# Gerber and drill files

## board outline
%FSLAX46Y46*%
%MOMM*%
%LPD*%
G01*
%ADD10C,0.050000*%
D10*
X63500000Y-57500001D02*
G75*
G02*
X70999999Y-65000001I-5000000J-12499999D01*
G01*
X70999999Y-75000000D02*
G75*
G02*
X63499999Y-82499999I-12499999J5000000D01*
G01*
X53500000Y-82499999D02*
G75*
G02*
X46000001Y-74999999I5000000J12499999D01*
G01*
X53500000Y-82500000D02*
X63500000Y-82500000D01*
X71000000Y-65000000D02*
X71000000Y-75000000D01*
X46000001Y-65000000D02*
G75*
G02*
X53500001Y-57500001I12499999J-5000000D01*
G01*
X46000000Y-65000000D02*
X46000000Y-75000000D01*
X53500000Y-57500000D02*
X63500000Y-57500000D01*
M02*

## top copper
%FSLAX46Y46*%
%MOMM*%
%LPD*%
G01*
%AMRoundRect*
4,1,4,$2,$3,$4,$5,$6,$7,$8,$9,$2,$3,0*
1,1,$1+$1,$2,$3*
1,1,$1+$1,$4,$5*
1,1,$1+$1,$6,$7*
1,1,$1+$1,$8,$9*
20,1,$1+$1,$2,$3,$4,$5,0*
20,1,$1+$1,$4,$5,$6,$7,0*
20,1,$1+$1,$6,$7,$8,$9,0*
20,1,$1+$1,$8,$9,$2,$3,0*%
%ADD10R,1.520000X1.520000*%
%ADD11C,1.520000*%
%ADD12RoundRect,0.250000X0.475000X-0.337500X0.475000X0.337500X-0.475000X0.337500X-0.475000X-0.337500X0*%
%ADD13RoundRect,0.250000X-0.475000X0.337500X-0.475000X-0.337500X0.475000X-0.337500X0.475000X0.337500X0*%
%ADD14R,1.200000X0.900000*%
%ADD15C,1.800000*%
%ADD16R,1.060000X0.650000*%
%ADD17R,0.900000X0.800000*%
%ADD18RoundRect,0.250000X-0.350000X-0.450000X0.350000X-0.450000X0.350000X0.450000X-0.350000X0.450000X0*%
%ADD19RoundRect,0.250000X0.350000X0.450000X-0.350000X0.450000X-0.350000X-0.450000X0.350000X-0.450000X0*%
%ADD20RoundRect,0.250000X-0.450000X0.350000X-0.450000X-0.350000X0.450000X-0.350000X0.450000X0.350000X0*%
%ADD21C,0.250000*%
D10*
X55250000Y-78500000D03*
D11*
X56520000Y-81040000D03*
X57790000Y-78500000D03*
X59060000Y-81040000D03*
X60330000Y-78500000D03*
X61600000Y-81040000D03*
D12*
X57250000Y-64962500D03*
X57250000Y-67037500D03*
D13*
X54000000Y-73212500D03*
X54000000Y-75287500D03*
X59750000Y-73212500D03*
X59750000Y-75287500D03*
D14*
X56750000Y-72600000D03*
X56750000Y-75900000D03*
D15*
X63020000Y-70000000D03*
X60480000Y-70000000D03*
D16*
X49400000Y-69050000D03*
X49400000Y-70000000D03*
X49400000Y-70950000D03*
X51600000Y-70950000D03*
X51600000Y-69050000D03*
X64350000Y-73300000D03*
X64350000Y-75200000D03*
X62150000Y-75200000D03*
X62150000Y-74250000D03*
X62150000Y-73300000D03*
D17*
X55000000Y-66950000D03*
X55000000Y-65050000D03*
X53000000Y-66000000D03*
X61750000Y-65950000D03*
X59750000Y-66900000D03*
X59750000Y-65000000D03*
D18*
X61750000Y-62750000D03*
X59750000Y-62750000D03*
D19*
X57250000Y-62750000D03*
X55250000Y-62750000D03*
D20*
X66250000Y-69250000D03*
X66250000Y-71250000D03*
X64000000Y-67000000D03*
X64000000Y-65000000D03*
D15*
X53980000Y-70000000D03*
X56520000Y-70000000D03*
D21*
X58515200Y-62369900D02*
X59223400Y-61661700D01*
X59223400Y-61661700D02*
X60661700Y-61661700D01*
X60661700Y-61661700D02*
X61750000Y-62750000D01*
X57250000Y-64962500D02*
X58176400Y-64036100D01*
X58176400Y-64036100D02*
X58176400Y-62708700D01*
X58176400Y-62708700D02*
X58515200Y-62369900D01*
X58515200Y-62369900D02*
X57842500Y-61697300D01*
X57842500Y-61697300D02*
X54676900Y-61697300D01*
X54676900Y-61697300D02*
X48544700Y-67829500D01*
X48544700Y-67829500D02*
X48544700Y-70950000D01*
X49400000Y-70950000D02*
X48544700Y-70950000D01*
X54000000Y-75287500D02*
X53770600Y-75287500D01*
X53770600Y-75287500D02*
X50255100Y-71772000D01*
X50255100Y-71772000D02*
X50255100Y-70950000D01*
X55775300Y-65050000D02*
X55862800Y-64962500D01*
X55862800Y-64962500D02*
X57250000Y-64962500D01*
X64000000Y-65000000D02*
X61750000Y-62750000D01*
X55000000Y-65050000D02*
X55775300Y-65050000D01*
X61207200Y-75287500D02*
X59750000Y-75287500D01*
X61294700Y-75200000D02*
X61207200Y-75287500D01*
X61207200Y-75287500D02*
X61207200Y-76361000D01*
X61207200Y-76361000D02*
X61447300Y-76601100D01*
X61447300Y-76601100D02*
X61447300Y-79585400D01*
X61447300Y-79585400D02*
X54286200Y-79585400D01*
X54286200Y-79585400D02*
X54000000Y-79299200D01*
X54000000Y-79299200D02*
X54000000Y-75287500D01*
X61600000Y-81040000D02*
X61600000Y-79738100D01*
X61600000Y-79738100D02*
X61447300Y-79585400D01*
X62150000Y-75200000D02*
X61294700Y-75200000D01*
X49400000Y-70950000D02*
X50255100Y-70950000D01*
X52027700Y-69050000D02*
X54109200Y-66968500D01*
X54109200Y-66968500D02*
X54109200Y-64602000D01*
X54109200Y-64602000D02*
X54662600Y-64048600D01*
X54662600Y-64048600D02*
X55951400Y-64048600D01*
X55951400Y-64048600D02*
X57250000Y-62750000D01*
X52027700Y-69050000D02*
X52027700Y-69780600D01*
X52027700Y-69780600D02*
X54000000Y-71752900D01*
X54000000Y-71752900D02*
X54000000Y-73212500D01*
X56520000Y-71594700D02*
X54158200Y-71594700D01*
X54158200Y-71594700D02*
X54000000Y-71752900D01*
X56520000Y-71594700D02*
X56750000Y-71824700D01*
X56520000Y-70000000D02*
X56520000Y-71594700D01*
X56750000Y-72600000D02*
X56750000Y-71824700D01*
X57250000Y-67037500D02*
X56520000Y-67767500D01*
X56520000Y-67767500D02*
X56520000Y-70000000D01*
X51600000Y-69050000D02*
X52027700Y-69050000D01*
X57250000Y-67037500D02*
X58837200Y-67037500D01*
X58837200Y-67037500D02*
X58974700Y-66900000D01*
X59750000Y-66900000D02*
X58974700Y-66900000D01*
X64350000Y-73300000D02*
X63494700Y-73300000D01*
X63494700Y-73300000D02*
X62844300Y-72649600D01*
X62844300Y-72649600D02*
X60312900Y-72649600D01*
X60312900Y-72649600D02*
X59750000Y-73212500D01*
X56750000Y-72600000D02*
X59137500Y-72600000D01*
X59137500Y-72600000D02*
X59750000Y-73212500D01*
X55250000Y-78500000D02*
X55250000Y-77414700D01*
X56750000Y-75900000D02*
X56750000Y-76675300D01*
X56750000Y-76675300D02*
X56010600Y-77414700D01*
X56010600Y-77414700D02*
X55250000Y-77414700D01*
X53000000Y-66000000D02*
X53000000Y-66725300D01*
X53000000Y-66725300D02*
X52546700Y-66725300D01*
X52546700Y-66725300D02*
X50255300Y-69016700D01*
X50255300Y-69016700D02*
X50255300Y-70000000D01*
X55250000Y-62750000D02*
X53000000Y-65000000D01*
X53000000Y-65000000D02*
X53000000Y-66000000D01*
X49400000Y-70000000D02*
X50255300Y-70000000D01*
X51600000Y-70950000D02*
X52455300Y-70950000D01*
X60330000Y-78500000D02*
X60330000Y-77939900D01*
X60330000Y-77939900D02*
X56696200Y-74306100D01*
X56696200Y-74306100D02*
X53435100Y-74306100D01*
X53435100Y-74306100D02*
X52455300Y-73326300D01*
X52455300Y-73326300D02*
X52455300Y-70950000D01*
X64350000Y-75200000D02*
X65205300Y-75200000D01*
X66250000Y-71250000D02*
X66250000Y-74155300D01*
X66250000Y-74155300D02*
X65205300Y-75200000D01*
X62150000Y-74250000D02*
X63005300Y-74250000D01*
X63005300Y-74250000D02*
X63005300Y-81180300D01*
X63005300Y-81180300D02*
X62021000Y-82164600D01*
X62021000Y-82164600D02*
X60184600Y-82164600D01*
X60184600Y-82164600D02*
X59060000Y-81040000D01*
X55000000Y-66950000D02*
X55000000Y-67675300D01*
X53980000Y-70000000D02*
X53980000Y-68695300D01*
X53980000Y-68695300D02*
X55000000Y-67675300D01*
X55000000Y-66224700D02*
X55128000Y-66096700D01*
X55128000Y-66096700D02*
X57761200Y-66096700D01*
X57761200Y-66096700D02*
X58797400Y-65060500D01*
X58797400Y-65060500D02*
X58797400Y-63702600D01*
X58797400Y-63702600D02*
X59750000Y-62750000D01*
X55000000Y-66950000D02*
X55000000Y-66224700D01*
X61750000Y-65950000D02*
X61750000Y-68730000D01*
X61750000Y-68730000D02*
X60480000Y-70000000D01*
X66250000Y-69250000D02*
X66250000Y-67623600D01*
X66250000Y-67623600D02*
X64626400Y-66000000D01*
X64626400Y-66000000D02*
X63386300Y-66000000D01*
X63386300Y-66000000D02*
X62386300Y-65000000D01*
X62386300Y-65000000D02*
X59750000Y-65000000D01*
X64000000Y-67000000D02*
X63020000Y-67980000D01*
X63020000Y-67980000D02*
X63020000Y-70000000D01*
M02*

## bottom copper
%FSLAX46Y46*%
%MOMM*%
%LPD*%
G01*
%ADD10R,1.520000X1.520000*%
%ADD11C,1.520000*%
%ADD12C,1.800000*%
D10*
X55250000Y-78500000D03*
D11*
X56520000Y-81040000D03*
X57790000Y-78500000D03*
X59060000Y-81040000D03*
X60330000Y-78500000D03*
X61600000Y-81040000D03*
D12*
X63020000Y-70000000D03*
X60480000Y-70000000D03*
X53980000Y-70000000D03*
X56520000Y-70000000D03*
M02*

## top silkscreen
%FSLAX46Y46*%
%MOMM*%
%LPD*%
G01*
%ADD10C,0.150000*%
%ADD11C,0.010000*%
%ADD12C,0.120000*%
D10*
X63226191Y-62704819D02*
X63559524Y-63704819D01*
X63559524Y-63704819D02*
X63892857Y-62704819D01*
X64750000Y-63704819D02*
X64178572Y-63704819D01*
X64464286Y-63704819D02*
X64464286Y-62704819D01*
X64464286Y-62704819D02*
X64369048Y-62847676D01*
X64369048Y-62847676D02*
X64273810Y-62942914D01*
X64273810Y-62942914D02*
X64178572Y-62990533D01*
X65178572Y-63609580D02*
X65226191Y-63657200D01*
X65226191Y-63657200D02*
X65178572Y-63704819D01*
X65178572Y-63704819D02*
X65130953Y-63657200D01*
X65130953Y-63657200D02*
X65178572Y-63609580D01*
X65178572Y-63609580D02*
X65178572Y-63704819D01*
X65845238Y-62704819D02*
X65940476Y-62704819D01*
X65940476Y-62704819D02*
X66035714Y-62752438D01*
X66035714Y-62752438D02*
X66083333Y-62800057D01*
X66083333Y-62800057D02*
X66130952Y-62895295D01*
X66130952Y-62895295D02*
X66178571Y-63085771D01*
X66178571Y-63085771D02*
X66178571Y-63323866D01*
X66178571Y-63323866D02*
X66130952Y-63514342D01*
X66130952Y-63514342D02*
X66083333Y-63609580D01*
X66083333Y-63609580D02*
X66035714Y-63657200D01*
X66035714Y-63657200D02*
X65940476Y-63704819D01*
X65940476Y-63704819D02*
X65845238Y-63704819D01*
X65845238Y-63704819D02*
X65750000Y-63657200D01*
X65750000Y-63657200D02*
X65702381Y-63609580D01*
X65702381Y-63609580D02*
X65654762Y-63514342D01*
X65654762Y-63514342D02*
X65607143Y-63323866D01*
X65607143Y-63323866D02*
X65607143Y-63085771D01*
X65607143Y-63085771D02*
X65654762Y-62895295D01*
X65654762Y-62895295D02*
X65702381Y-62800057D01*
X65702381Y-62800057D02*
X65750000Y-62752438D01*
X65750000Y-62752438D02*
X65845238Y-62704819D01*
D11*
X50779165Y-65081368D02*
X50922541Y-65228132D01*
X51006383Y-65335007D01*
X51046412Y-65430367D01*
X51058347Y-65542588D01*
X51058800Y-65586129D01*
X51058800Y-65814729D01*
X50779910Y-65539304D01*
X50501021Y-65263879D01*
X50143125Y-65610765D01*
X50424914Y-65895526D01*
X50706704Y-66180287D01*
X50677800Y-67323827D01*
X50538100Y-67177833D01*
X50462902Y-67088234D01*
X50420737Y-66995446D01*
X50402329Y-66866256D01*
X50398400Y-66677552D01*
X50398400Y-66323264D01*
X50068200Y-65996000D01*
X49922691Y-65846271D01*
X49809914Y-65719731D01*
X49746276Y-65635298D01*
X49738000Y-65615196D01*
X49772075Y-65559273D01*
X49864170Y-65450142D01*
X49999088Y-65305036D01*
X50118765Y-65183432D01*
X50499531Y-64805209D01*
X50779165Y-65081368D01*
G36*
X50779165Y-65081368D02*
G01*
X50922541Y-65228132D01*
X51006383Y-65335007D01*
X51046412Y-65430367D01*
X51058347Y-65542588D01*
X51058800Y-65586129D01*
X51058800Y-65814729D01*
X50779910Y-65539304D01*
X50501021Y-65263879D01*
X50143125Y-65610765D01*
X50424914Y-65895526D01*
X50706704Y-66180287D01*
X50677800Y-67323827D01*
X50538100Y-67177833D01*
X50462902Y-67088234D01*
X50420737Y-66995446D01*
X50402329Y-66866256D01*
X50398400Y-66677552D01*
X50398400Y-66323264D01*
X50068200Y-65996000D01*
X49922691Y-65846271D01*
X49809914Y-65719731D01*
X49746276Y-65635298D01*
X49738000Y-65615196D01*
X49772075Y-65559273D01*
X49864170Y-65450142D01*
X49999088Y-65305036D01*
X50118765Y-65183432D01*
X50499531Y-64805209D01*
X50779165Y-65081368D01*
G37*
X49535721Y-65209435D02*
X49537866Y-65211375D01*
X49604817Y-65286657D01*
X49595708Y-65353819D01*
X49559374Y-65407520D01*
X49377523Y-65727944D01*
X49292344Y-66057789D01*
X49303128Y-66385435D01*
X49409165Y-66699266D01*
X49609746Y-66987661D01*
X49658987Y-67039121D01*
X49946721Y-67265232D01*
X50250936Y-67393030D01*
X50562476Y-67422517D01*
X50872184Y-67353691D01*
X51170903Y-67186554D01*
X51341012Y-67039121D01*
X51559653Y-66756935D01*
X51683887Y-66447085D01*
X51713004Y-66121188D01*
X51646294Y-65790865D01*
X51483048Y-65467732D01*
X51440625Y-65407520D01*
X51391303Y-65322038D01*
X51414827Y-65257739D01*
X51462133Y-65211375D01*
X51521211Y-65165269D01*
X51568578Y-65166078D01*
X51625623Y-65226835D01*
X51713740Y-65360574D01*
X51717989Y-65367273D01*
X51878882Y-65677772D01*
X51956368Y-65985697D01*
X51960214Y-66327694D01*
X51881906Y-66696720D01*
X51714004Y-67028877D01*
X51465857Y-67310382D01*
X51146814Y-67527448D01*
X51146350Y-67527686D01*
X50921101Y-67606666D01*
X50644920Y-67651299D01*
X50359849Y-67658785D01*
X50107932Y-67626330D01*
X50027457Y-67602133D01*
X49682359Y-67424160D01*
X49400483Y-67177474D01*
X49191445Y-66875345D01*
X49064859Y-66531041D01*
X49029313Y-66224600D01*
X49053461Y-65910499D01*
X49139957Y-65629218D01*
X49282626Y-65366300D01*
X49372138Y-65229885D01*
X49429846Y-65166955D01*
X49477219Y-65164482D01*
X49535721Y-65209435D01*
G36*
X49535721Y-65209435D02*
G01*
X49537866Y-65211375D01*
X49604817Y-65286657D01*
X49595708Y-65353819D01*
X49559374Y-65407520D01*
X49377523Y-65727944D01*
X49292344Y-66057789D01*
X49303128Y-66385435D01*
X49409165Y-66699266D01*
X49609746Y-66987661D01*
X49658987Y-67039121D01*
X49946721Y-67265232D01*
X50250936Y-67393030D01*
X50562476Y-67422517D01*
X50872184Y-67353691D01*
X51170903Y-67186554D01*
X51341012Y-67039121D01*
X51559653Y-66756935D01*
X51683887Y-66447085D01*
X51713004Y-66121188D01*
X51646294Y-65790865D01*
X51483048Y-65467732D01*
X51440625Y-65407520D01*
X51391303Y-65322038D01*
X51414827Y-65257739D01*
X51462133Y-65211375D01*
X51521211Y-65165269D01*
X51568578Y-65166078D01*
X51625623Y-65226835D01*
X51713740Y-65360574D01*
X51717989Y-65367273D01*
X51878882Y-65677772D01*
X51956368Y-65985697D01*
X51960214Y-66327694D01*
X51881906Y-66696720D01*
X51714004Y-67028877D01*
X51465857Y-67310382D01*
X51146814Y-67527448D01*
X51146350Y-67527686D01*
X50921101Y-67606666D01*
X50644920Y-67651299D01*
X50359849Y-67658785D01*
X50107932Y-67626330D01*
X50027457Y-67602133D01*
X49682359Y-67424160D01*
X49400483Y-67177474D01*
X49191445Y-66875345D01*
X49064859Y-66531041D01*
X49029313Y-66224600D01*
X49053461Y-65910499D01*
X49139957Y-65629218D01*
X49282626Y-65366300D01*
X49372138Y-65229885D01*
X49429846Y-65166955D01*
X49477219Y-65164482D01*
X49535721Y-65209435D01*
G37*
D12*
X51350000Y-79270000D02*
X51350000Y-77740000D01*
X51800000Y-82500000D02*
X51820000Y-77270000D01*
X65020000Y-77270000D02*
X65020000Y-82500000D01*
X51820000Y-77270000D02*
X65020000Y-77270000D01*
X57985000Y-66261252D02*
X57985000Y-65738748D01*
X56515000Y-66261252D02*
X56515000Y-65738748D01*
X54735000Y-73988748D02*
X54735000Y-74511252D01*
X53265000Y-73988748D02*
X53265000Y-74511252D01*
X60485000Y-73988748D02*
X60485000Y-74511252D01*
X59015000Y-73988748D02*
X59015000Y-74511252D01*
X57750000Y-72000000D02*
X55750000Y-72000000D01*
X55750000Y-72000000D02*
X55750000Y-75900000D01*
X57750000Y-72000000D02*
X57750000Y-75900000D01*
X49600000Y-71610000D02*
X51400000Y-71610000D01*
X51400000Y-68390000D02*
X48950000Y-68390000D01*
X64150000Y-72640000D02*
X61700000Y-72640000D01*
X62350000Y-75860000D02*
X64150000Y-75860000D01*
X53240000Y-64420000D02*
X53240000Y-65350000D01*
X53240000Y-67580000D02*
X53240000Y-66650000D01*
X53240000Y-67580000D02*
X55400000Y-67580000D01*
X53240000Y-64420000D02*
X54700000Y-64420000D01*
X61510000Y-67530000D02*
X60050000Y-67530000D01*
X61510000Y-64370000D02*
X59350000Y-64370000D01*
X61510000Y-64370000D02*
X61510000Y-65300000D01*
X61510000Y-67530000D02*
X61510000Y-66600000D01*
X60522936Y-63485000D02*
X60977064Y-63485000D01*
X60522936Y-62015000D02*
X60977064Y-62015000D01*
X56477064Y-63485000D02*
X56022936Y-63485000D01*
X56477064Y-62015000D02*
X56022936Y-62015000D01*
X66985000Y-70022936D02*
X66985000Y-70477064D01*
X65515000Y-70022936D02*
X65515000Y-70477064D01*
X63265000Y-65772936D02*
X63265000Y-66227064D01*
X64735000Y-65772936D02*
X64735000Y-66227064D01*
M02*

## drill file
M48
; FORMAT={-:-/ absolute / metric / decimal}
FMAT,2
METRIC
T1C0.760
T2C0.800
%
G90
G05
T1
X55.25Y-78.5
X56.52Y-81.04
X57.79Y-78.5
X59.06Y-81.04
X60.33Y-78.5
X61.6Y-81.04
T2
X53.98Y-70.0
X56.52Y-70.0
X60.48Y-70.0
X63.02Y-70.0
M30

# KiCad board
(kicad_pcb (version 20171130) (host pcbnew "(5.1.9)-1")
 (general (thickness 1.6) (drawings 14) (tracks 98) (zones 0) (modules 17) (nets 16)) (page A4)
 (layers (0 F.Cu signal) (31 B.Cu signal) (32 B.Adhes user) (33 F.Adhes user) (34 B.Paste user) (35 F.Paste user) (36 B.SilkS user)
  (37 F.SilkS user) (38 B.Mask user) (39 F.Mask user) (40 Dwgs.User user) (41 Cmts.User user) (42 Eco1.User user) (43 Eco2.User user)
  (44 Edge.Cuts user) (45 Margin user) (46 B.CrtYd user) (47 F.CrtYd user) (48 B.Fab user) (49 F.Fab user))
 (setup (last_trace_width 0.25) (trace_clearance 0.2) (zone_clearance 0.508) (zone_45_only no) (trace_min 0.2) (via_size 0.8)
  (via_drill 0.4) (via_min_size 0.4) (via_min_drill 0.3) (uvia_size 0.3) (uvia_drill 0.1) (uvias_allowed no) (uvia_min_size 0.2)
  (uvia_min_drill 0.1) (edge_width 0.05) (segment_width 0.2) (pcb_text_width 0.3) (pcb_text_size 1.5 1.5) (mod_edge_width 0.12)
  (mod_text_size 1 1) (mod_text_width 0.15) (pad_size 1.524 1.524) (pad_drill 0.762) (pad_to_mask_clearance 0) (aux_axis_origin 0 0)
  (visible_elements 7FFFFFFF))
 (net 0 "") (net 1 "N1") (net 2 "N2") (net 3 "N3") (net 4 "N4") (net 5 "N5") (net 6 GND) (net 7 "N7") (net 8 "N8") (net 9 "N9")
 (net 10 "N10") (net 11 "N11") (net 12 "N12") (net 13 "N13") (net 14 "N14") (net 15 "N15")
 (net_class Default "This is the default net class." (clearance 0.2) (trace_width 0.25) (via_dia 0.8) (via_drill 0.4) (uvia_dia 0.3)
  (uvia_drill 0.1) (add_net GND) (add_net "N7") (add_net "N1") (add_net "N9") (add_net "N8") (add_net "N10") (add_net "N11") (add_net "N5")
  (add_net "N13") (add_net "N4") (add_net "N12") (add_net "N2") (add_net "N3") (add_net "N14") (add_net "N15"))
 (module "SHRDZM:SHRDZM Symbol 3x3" (layer F.Cu) (at 50.5 66.25)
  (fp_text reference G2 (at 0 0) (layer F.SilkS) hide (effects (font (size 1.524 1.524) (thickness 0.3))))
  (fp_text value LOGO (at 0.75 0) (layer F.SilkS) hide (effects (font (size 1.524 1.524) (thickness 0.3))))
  (fp_poly
   (pts (xy 0.279165 -1.168632) (xy 0.422541 -1.021868) (xy 0.506383 -0.914993) (xy 0.546412 -0.819633) (xy 0.558347 -0.707412)
    (xy 0.5588 -0.663871) (xy 0.5588 -0.435271) (xy 0.27991 -0.710696) (xy 0.001021 -0.986121) (xy -0.356875 -0.639235)
    (xy -0.075086 -0.354474) (xy 0.206704 -0.069713) (xy 0.1778 1.073827) (xy 0.0381 0.927833) (xy -0.037098 0.838234)
    (xy -0.079263 0.745446) (xy -0.097671 0.616256) (xy -0.1016 0.427552) (xy -0.1016 0.073264) (xy -0.4318 -0.254) (xy -0.577309 -0.403729)
    (xy -0.690086 -0.530269) (xy -0.753724 -0.614702) (xy -0.762 -0.634804) (xy -0.727925 -0.690727) (xy -0.63583 -0.799858)
    (xy -0.500912 -0.944964) (xy -0.381235 -1.066568) (xy -0.000469 -1.444791) (xy 0.279165 -1.168632))
   (layer F.SilkS) (width 0.01))
  (fp_poly
   (pts (xy -0.964279 -1.040565) (xy -0.962134 -1.038625) (xy -0.895183 -0.963343) (xy -0.904292 -0.896181) (xy -0.940626 -0.84248)
    (xy -1.122477 -0.522056) (xy -1.207656 -0.192211) (xy -1.196872 0.135435) (xy -1.090835 0.449266) (xy -0.890254 0.737661)
    (xy -0.841013 0.789121) (xy -0.553279 1.015232) (xy -0.249064 1.14303) (xy 0.062476 1.172517) (xy 0.372184 1.103691)
    (xy 0.670903 0.936554) (xy 0.841012 0.789121) (xy 1.059653 0.506935) (xy 1.183887 0.197085) (xy 1.213004 -0.128812)
    (xy 1.146294 -0.459135) (xy 0.983048 -0.782268) (xy 0.940625 -0.84248) (xy 0.891303 -0.927962) (xy 0.914827 -0.992261)
    (xy 0.962133 -1.038625) (xy 1.021211 -1.084731) (xy 1.068578 -1.083922) (xy 1.125623 -1.023165) (xy 1.21374 -0.889426)
    (xy 1.217989 -0.882727) (xy 1.378882 -0.572228) (xy 1.456368 -0.264303) (xy 1.460214 0.077694) (xy 1.381906 0.44672)
    (xy 1.214004 0.778877) (xy 0.965857 1.060382) (xy 0.646814 1.277448) (xy 0.64635 1.277686) (xy 0.421101 1.356666) (xy 0.14492 1.401299)
    (xy -0.140151 1.408785) (xy -0.392068 1.37633) (xy -0.472543 1.352133) (xy -0.817641 1.17416) (xy -1.099517 0.927474)
    (xy -1.308555 0.625345) (xy -1.435141 0.281041) (xy -1.470687 -0.0254) (xy -1.446539 -0.339501) (xy -1.360043 -0.620782)
    (xy -1.217374 -0.8837) (xy -1.127862 -1.020115) (xy -1.070154 -1.083045) (xy -1.022781 -1.085518) (xy -0.964279 -1.040565))
   (layer F.SilkS) (width 0.01)))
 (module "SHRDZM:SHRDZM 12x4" (layer B.Cu) (at 58.75 63.25 180)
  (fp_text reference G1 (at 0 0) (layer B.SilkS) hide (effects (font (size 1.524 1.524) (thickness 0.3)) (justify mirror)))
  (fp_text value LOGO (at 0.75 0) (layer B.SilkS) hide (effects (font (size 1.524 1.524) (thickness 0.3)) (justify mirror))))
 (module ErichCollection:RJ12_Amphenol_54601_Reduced (layer F.Cu) (at 55.25 78.5)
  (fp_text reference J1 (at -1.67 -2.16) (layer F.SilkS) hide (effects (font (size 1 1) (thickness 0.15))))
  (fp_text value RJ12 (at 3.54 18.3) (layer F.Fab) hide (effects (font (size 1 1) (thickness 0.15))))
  (fp_line (start -3.9 0.77) (end -3.9 -0.76) (layer F.SilkS) (width 0.12))
  (fp_line (start -3.45 4) (end -3.43 -1.23) (layer F.SilkS) (width 0.12))
  (fp_line (start 9.77 -1.23) (end 9.77 4) (layer F.SilkS) (width 0.12))
  (fp_line (start -3.43 -1.23) (end 9.77 -1.23) (layer F.SilkS) (width 0.12))
  (pad 1 thru_hole rect (at 0 0) (size 1.52 1.52) (drill 0.76) (layers *.Cu *.Mask) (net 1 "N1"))
  (pad 2 thru_hole circle (at 1.27 2.54) (size 1.52 1.52) (drill 0.76) (layers *.Cu *.Mask) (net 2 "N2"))
  (pad 3 thru_hole circle (at 2.54 0) (size 1.52 1.52) (drill 0.76) (layers *.Cu *.Mask) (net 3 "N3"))
  (pad 4 thru_hole circle (at 3.81 2.54) (size 1.52 1.52) (drill 0.76) (layers *.Cu *.Mask) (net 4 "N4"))
  (pad 5 thru_hole circle (at 5.08 0) (size 1.52 1.52) (drill 0.76) (layers *.Cu *.Mask) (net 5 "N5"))
  (pad 6 thru_hole circle (at 6.35 2.54) (size 1.52 1.52) (drill 0.76) (layers *.Cu *.Mask) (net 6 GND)))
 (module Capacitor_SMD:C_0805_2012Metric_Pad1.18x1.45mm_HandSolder (layer F.Cu) (at 57.25 66 90)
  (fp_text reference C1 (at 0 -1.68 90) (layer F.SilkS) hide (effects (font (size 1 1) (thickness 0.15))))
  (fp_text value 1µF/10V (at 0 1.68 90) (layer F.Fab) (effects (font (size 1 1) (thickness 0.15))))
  (fp_line (start -0.261252 0.735) (end 0.261252 0.735) (layer F.SilkS) (width 0.12))
  (fp_line (start -0.261252 -0.735) (end 0.261252 -0.735) (layer F.SilkS) (width 0.12))
  (pad 2 smd roundrect (at 1.0375 0 90) (size 1.175 1.45) (layers F.Cu F.Paste F.Mask) (roundrect_rratio 0.212766) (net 6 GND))
  (pad 1 smd roundrect (at -1.0375 0 90) (size 1.175 1.45) (layers F.Cu F.Paste F.Mask) (roundrect_rratio 0.212766) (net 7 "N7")))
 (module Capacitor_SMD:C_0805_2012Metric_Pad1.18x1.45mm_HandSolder (layer F.Cu) (at 54 74.25 270)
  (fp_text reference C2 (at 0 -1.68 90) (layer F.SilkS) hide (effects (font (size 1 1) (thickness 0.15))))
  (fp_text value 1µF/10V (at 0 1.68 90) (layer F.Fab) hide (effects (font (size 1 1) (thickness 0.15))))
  (fp_line (start -0.261252 -0.735) (end 0.261252 -0.735) (layer F.SilkS) (width 0.12))
  (fp_line (start -0.261252 0.735) (end 0.261252 0.735) (layer F.SilkS) (width 0.12))
  (pad 1 smd roundrect (at -1.0375 0 270) (size 1.175 1.45) (layers F.Cu F.Paste F.Mask) (roundrect_rratio 0.212766) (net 7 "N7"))
  (pad 2 smd roundrect (at 1.0375 0 270) (size 1.175 1.45) (layers F.Cu F.Paste F.Mask) (roundrect_rratio 0.212766) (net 6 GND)))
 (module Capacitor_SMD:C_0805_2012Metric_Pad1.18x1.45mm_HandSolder (layer F.Cu) (at 59.75 74.25 270)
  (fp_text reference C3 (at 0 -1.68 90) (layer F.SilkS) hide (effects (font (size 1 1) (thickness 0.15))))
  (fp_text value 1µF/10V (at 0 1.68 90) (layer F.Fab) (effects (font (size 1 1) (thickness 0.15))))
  (fp_line (start -0.261252 -0.735) (end 0.261252 -0.735) (layer F.SilkS) (width 0.12))
  (fp_line (start -0.261252 0.735) (end 0.261252 0.735) (layer F.SilkS) (width 0.12))
  (pad 1 smd roundrect (at -1.0375 0 270) (size 1.175 1.45) (layers F.Cu F.Paste F.Mask) (roundrect_rratio 0.212766) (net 7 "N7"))
  (pad 2 smd roundrect (at 1.0375 0 270) (size 1.175 1.45) (layers F.Cu F.Paste F.Mask) (roundrect_rratio 0.212766) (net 6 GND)))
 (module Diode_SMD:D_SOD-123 (layer F.Cu) (at 56.75 74.25 270)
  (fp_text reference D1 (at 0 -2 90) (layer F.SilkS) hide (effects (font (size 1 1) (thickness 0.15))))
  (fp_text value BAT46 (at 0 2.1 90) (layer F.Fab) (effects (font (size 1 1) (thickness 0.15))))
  (fp_line (start -2.25 -1) (end -2.25 1) (layer F.SilkS) (width 0.12))
  (fp_line (start -2.25 1) (end 1.65 1) (layer F.SilkS) (width 0.12))
  (fp_line (start -2.25 -1) (end 1.65 -1) (layer F.SilkS) (width 0.12))
  (pad 1 smd rect (at -1.65 0 270) (size 0.9 1.2) (layers F.Cu F.Paste F.Mask) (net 7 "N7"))
  (pad 2 smd rect (at 1.65 0 270) (size 0.9 1.2) (layers F.Cu F.Paste F.Mask) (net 1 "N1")))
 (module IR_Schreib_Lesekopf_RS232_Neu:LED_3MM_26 (layer F.Cu) (at 61.75 70 180)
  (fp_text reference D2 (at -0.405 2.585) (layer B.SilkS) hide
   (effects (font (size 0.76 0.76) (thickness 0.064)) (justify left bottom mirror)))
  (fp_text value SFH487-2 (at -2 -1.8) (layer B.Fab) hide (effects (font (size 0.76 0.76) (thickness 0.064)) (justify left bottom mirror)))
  (pad 2 thru_hole circle (at -1.27 0 180) (size 1.8 1.8) (drill 0.8) (layers *.Cu *.Mask) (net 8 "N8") (solder_mask_margin 0.1016))
  (pad 1 thru_hole circle (at 1.27 0 180) (size 1.8 1.8) (drill 0.8) (layers *.Cu *.Mask) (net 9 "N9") (solder_mask_margin 0.1016)))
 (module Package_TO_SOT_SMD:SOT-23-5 (layer F.Cu) (at 50.5 70)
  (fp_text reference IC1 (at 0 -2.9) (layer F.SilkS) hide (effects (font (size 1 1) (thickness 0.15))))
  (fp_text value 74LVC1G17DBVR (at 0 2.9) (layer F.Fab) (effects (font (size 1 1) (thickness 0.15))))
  (fp_line (start -0.9 1.61) (end 0.9 1.61) (layer F.SilkS) (width 0.12))
  (fp_line (start 0.9 -1.61) (end -1.55 -1.61) (layer F.SilkS) (width 0.12))
  (pad 1 smd rect (at -1.1 -0.95) (size 1.06 0.65) (layers F.Cu F.Paste F.Mask) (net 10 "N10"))
  (pad 2 smd rect (at -1.1 0) (size 1.06 0.65) (layers F.Cu F.Paste F.Mask) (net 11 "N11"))
  (pad 3 smd rect (at -1.1 0.95) (size 1.06 0.65) (layers F.Cu F.Paste F.Mask) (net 6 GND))
  (pad 4 smd rect (at 1.1 0.95) (size 1.06 0.65) (layers F.Cu F.Paste F.Mask) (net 5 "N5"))
  (pad 5 smd rect (at 1.1 -0.95) (size 1.06 0.65) (layers F.Cu F.Paste F.Mask) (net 7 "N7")))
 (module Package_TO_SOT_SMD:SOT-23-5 (layer F.Cu) (at 63.25 74.25)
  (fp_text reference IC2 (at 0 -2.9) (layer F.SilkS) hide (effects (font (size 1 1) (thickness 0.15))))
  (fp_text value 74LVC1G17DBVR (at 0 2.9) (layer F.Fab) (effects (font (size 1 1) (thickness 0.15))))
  (fp_line (start 0.9 -1.61) (end -1.55 -1.61) (layer F.SilkS) (width 0.12))
  (fp_line (start -0.9 1.61) (end 0.9 1.61) (layer F.SilkS) (width 0.12))
  (pad 5 smd rect (at 1.1 -0.95) (size 1.06 0.65) (layers F.Cu F.Paste F.Mask) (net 7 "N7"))
  (pad 4 smd rect (at 1.1 0.95) (size 1.06 0.65) (layers F.Cu F.Paste F.Mask) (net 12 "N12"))
  (pad 3 smd rect (at -1.1 0.95) (size 1.06 0.65) (layers F.Cu F.Paste F.Mask) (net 6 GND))
  (pad 2 smd rect (at -1.1 0) (size 1.06 0.65) (layers F.Cu F.Paste F.Mask) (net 4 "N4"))
  (pad 1 smd rect (at -1.1 -0.95) (size 1.06 0.65) (layers F.Cu F.Paste F.Mask) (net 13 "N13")))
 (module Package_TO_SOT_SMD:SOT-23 (layer F.Cu) (at 54 66 180)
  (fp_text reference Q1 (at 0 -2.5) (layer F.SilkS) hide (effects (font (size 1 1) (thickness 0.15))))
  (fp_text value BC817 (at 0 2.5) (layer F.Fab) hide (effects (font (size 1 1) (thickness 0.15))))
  (fp_line (start 0.76 1.58) (end 0.76 0.65) (layer F.SilkS) (width 0.12))
  (fp_line (start 0.76 -1.58) (end 0.76 -0.65) (layer F.SilkS) (width 0.12))
  (fp_line (start 0.76 -1.58) (end -1.4 -1.58) (layer F.SilkS) (width 0.12))
  (fp_line (start 0.76 1.58) (end -0.7 1.58) (layer F.SilkS) (width 0.12))
  (pad 1 smd rect (at -1 -0.95 180) (size 0.9 0.8) (layers F.Cu F.Paste F.Mask) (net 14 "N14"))
  (pad 2 smd rect (at -1 0.95 180) (size 0.9 0.8) (layers F.Cu F.Paste F.Mask) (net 6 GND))
  (pad 3 smd rect (at 1 0 180) (size 0.9 0.8) (layers F.Cu F.Paste F.Mask) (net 11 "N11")))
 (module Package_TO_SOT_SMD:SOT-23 (layer F.Cu) (at 60.75 65.95)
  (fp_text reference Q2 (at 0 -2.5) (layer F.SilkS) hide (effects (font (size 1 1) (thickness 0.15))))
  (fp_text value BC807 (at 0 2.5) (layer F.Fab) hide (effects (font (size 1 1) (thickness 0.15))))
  (fp_line (start 0.76 1.58) (end -0.7 1.58) (layer F.SilkS) (width 0.12))
  (fp_line (start 0.76 -1.58) (end -1.4 -1.58) (layer F.SilkS) (width 0.12))
  (fp_line (start 0.76 -1.58) (end 0.76 -0.65) (layer F.SilkS) (width 0.12))
  (fp_line (start 0.76 1.58) (end 0.76 0.65) (layer F.SilkS) (width 0.12))
  (pad 3 smd rect (at 1 0) (size 0.9 0.8) (layers F.Cu F.Paste F.Mask) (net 9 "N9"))
  (pad 2 smd rect (at -1 0.95) (size 0.9 0.8) (layers F.Cu F.Paste F.Mask) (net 7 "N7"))
  (pad 1 smd rect (at -1 -0.95) (size 0.9 0.8) (layers F.Cu F.Paste F.Mask) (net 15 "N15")))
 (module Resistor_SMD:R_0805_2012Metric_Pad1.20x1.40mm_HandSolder (layer F.Cu) (at 60.75 62.75)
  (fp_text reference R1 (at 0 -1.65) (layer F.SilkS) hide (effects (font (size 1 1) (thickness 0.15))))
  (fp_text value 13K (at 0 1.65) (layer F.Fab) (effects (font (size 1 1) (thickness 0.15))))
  (fp_line (start -0.227064 0.735) (end 0.227064 0.735) (layer F.SilkS) (width 0.12))
  (fp_line (start -0.227064 -0.735) (end 0.227064 -0.735) (layer F.SilkS) (width 0.12))
  (pad 2 smd roundrect (at 1 0) (size 1.2 1.4) (layers F.Cu F.Paste F.Mask) (roundrect_rratio 0.208333) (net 6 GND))
  (pad 1 smd roundrect (at -1 0) (size 1.2 1.4) (layers F.Cu F.Paste F.Mask) (roundrect_rratio 0.208333) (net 14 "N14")))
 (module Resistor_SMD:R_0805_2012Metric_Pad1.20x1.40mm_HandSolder (layer F.Cu) (at 56.25 62.75 180)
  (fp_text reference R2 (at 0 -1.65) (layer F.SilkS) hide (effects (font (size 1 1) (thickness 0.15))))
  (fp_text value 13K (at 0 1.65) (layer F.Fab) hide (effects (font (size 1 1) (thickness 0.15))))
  (fp_line (start -0.227064 -0.735) (end 0.227064 -0.735) (layer F.SilkS) (width 0.12))
  (fp_line (start -0.227064 0.735) (end 0.227064 0.735) (layer F.SilkS) (width 0.12))
  (pad 1 smd roundrect (at -1 0 180) (size 1.2 1.4) (layers F.Cu F.Paste F.Mask) (roundrect_rratio 0.208333) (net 7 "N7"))
  (pad 2 smd roundrect (at 1 0 180) (size 1.2 1.4) (layers F.Cu F.Paste F.Mask) (roundrect_rratio 0.208333) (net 11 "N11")))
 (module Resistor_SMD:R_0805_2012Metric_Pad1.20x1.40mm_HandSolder (layer F.Cu) (at 66.25 70.25 270)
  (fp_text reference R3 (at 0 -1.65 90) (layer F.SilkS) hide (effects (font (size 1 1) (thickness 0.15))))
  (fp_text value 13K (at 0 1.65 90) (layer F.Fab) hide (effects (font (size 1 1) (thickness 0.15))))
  (fp_line (start -0.227064 -0.735) (end 0.227064 -0.735) (layer F.SilkS) (width 0.12))
  (fp_line (start -0.227064 0.735) (end 0.227064 0.735) (layer F.SilkS) (width 0.12))
  (pad 1 smd roundrect (at -1 0 270) (size 1.2 1.4) (layers F.Cu F.Paste F.Mask) (roundrect_rratio 0.208333) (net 15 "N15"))
  (pad 2 smd roundrect (at 1 0 270) (size 1.2 1.4) (layers F.Cu F.Paste F.Mask) (roundrect_rratio 0.208333) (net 12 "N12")))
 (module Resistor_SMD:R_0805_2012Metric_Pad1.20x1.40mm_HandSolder (layer F.Cu) (at 64 66 270)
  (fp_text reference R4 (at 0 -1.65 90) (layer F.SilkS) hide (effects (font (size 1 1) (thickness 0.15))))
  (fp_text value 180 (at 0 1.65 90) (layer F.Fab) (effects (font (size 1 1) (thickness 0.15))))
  (fp_line (start -0.227064 0.735) (end 0.227064 0.735) (layer F.SilkS) (width 0.12))
  (fp_line (start -0.227064 -0.735) (end 0.227064 -0.735) (layer F.SilkS) (width 0.12))
  (pad 2 smd roundrect (at 1 0 270) (size 1.2 1.4) (layers F.Cu F.Paste F.Mask) (roundrect_rratio 0.208333) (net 8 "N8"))
  (pad 1 smd roundrect (at -1 0 270) (size 1.2 1.4) (layers F.Cu F.Paste F.Mask) (roundrect_rratio 0.208333) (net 6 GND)))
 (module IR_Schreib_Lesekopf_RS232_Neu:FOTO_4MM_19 (layer B.Cu) (at 55.25 70)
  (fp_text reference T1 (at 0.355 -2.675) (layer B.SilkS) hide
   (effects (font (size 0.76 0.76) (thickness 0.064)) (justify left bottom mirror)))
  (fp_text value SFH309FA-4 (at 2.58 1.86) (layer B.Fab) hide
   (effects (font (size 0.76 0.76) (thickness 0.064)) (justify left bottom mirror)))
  (pad 1 thru_hole circle (at -1.27 0) (size 1.8 1.8) (drill 0.8) (layers *.Cu *.Mask) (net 14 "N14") (solder_mask_margin 0.1016))
  (pad 2 thru_hole circle (at 1.27 0) (size 1.8 1.8) (drill 0.8) (layers *.Cu *.Mask) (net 7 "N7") (solder_mask_margin 0.1016)))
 (gr_arc (start 58.5 70) (end 70.999999 65.000001) (angle -46.39718103) (layer Edge.Cuts) (width 0.05))
 (gr_arc (start 58.5 70) (end 63.499999 82.499999) (angle -46.39718103) (layer Edge.Cuts) (width 0.05))
 (gr_arc (start 58.5 70) (end 46.000001 74.999999) (angle -46.39718103) (layer Edge.Cuts) (width 0.05))
 (gr_line (start 53.5 82.5) (end 63.5 82.5) (layer Edge.Cuts) (width 0.05))
 (gr_line (start 71 65) (end 71 75) (layer Edge.Cuts) (width 0.05))
 (gr_arc (start 58.5 70) (end 53.500001 57.500001) (angle -46.39718103) (layer Edge.Cuts) (width 0.05))
 (gr_line (start 46 65) (end 46 75) (layer Edge.Cuts) (width 0.05))
 (gr_line (start 53.5 57.5) (end 63.5 57.5) (layer Edge.Cuts) (width 0.05))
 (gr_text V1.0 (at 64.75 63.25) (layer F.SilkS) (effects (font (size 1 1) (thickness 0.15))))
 (segment (start 58.5152 62.3699) (end 59.2234 61.6617) (width 0.25) (layer F.Cu) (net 6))
 (segment (start 59.2234 61.6617) (end 60.6617 61.6617) (width 0.25) (layer F.Cu) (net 6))
 (segment (start 60.6617 61.6617) (end 61.75 62.75) (width 0.25) (layer F.Cu) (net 6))
 (segment (start 57.25 64.9625) (end 58.1764 64.0361) (width 0.25) (layer F.Cu) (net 6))
 (segment (start 58.1764 64.0361) (end 58.1764 62.7087) (width 0.25) (layer F.Cu) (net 6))
 (segment (start 58.1764 62.7087) (end 58.5152 62.3699) (width 0.25) (layer F.Cu) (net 6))
 (segment (start 58.5152 62.3699) (end 57.8425 61.6973) (width 0.25) (layer F.Cu) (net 6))
 (segment (start 57.8425 61.6973) (end 54.6769 61.6973) (width 0.25) (layer F.Cu) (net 6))
 (segment (start 54.6769 61.6973) (end 48.5447 67.8295) (width 0.25) (layer F.Cu) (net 6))
 (segment (start 48.5447 67.8295) (end 48.5447 70.95) (width 0.25) (layer F.Cu) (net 6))
 (segment (start 49.4 70.95) (end 48.5447 70.95) (width 0.25) (layer F.Cu) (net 6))
 (segment (start 54 75.2875) (end 53.7706 75.2875) (width 0.25) (layer F.Cu) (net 6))
 (segment (start 53.7706 75.2875) (end 50.2551 71.772) (width 0.25) (layer F.Cu) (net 6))
 (segment (start 50.2551 71.772) (end 50.2551 70.95) (width 0.25) (layer F.Cu) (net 6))
 (segment (start 55.7753 65.05) (end 55.8628 64.9625) (width 0.25) (layer F.Cu) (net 6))
 (segment (start 55.8628 64.9625) (end 57.25 64.9625) (width 0.25) (layer F.Cu) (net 6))
 (segment (start 64 65) (end 61.75 62.75) (width 0.25) (layer F.Cu) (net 6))
 (segment (start 55 65.05) (end 55.7753 65.05) (width 0.25) (layer F.Cu) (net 6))
 (segment (start 61.2072 75.2875) (end 59.75 75.2875) (width 0.25) (layer F.Cu) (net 6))
 (segment (start 61.2947 75.2) (end 61.2072 75.2875) (width 0.25) (layer F.Cu) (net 6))
 (segment (start 61.2072 75.2875) (end 61.2072 76.361) (width 0.25) (layer F.Cu) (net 6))
 (segment (start 61.2072 76.361) (end 61.4473 76.6011) (width 0.25) (layer F.Cu) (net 6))
 (segment (start 61.4473 76.6011) (end 61.4473 79.5854) (width 0.25) (layer F.Cu) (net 6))
 (segment (start 61.4473 79.5854) (end 54.2862 79.5854) (width 0.25) (layer F.Cu) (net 6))
 (segment (start 54.2862 79.5854) (end 54 79.2992) (width 0.25) (layer F.Cu) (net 6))
 (segment (start 54 79.2992) (end 54 75.2875) (width 0.25) (layer F.Cu) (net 6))
 (segment (start 61.6 81.04) (end 61.6 79.7381) (width 0.25) (layer F.Cu) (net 6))
 (segment (start 61.6 79.7381) (end 61.4473 79.5854) (width 0.25) (layer F.Cu) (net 6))
 (segment (start 62.15 75.2) (end 61.2947 75.2) (width 0.25) (layer F.Cu) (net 6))
 (segment (start 49.4 70.95) (end 50.2551 70.95) (width 0.25) (layer F.Cu) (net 6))
 (segment (start 52.0277 69.05) (end 54.1092 66.9685) (width 0.25) (layer F.Cu) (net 7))
 (segment (start 54.1092 66.9685) (end 54.1092 64.602) (width 0.25) (layer F.Cu) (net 7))
 (segment (start 54.1092 64.602) (end 54.6626 64.0486) (width 0.25) (layer F.Cu) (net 7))
 (segment (start 54.6626 64.0486) (end 55.9514 64.0486) (width 0.25) (layer F.Cu) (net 7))
 (segment (start 55.9514 64.0486) (end 57.25 62.75) (width 0.25) (layer F.Cu) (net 7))
 (segment (start 52.0277 69.05) (end 52.0277 69.7806) (width 0.25) (layer F.Cu) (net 7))
 (segment (start 52.0277 69.7806) (end 54 71.7529) (width 0.25) (layer F.Cu) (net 7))
 (segment (start 54 71.7529) (end 54 73.2125) (width 0.25) (layer F.Cu) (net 7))
 (segment (start 56.52 71.5947) (end 54.1582 71.5947) (width 0.25) (layer F.Cu) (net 7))
 (segment (start 54.1582 71.5947) (end 54 71.7529) (width 0.25) (layer F.Cu) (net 7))
 (segment (start 56.52 71.5947) (end 56.75 71.8247) (width 0.25) (layer F.Cu) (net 7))
 (segment (start 56.52 70) (end 56.52 71.5947) (width 0.25) (layer F.Cu) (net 7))
 (segment (start 56.75 72.6) (end 56.75 71.8247) (width 0.25) (layer F.Cu) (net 7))
 (segment (start 57.25 67.0375) (end 56.52 67.7675) (width 0.25) (layer F.Cu) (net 7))
 (segment (start 56.52 67.7675) (end 56.52 70) (width 0.25) (layer F.Cu) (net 7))
 (segment (start 51.6 69.05) (end 52.0277 69.05) (width 0.25) (layer F.Cu) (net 7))
 (segment (start 57.25 67.0375) (end 58.8372 67.0375) (width 0.25) (layer F.Cu) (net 7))
 (segment (start 58.8372 67.0375) (end 58.9747 66.9) (width 0.25) (layer F.Cu) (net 7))
 (segment (start 59.75 66.9) (end 58.9747 66.9) (width 0.25) (layer F.Cu) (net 7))
 (segment (start 64.35 73.3) (end 63.4947 73.3) (width 0.25) (layer F.Cu) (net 7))
 (segment (start 63.4947 73.3) (end 62.8443 72.6496) (width 0.25) (layer F.Cu) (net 7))
 (segment (start 62.8443 72.6496) (end 60.3129 72.6496) (width 0.25) (layer F.Cu) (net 7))
 (segment (start 60.3129 72.6496) (end 59.75 73.2125) (width 0.25) (layer F.Cu) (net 7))
 (segment (start 56.75 72.6) (end 59.1375 72.6) (width 0.25) (layer F.Cu) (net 7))
 (segment (start 59.1375 72.6) (end 59.75 73.2125) (width 0.25) (layer F.Cu) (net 7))
 (segment (start 55.25 78.5) (end 55.25 77.4147) (width 0.25) (layer F.Cu) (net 1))
 (segment (start 56.75 75.9) (end 56.75 76.6753) (width 0.25) (layer F.Cu) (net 1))
 (segment (start 56.75 76.6753) (end 56.0106 77.4147) (width 0.25) (layer F.Cu) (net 1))
 (segment (start 56.0106 77.4147) (end 55.25 77.4147) (width 0.25) (layer F.Cu) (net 1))
 (segment (start 53 66) (end 53 66.7253) (width 0.25) (layer F.Cu) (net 11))
 (segment (start 53 66.7253) (end 52.5467 66.7253) (width 0.25) (layer F.Cu) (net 11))
 (segment (start 52.5467 66.7253) (end 50.2553 69.0167) (width 0.25) (layer F.Cu) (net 11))
 (segment (start 50.2553 69.0167) (end 50.2553 70) (width 0.25) (layer F.Cu) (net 11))
 (segment (start 55.25 62.75) (end 53 65) (width 0.25) (layer F.Cu) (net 11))
 (segment (start 53 65) (end 53 66) (width 0.25) (layer F.Cu) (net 11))
 (segment (start 49.4 70) (end 50.2553 70) (width 0.25) (layer F.Cu) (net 11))
 (segment (start 51.6 70.95) (end 52.4553 70.95) (width 0.25) (layer F.Cu) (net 5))
 (segment (start 60.33 78.5) (end 60.33 77.9399) (width 0.25) (layer F.Cu) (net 5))
 (segment (start 60.33 77.9399) (end 56.6962 74.3061) (width 0.25) (layer F.Cu) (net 5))
 (segment (start 56.6962 74.3061) (end 53.4351 74.3061) (width 0.25) (layer F.Cu) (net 5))
 (segment (start 53.4351 74.3061) (end 52.4553 73.3263) (width 0.25) (layer F.Cu) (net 5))
 (segment (start 52.4553 73.3263) (end 52.4553 70.95) (width 0.25) (layer F.Cu) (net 5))
 (segment (start 64.35 75.2) (end 65.2053 75.2) (width 0.25) (layer F.Cu) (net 12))
 (segment (start 66.25 71.25) (end 66.25 74.1553) (width 0.25) (layer F.Cu) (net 12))
 (segment (start 66.25 74.1553) (end 65.2053 75.2) (width 0.25) (layer F.Cu) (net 12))
 (segment (start 62.15 74.25) (end 63.0053 74.25) (width 0.25) (layer F.Cu) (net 4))
 (segment (start 63.0053 74.25) (end 63.0053 81.1803) (width 0.25) (layer F.Cu) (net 4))
 (segment (start 63.0053 81.1803) (end 62.021 82.1646) (width 0.25) (layer F.Cu) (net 4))
 (segment (start 62.021 82.1646) (end 60.1846 82.1646) (width 0.25) (layer F.Cu) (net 4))
 (segment (start 60.1846 82.1646) (end 59.06 81.04) (width 0.25) (layer F.Cu) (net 4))
 (segment (start 55 66.95) (end 55 67.6753) (width 0.25) (layer F.Cu) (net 14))
 (segment (start 53.98 70) (end 53.98 68.6953) (width 0.25) (layer F.Cu) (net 14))
 (segment (start 53.98 68.6953) (end 55 67.6753) (width 0.25) (layer F.Cu) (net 14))
 (segment (start 55 66.2247) (end 55.128 66.0967) (width 0.25) (layer F.Cu) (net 14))
 (segment (start 55.128 66.0967) (end 57.7612 66.0967) (width 0.25) (layer F.Cu) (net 14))
 (segment (start 57.7612 66.0967) (end 58.7974 65.0605) (width 0.25) (layer F.Cu) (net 14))
 (segment (start 58.7974 65.0605) (end 58.7974 63.7026) (width 0.25) (layer F.Cu) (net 14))
 (segment (start 58.7974 63.7026) (end 59.75 62.75) (width 0.25) (layer F.Cu) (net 14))
 (segment (start 55 66.95) (end 55 66.2247) (width 0.25) (layer F.Cu) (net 14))
 (segment (start 61.75 65.95) (end 61.75 68.73) (width 0.25) (layer F.Cu) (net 9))
 (segment (start 61.75 68.73) (end 60.48 70) (width 0.25) (layer F.Cu) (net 9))
 (segment (start 66.25 69.25) (end 66.25 67.6236) (width 0.25) (layer F.Cu) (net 15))
 (segment (start 66.25 67.6236) (end 64.6264 66) (width 0.25) (layer F.Cu) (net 15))
 (segment (start 64.6264 66) (end 63.3863 66) (width 0.25) (layer F.Cu) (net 15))
 (segment (start 63.3863 66) (end 62.3863 65) (width 0.25) (layer F.Cu) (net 15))
 (segment (start 62.3863 65) (end 59.75 65) (width 0.25) (layer F.Cu) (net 15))
 (segment (start 64 67) (end 63.02 67.98) (width 0.25) (layer F.Cu) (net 8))
 (segment (start 63.02 67.98) (end 63.02 70) (width 0.25) (layer F.Cu) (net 8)))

